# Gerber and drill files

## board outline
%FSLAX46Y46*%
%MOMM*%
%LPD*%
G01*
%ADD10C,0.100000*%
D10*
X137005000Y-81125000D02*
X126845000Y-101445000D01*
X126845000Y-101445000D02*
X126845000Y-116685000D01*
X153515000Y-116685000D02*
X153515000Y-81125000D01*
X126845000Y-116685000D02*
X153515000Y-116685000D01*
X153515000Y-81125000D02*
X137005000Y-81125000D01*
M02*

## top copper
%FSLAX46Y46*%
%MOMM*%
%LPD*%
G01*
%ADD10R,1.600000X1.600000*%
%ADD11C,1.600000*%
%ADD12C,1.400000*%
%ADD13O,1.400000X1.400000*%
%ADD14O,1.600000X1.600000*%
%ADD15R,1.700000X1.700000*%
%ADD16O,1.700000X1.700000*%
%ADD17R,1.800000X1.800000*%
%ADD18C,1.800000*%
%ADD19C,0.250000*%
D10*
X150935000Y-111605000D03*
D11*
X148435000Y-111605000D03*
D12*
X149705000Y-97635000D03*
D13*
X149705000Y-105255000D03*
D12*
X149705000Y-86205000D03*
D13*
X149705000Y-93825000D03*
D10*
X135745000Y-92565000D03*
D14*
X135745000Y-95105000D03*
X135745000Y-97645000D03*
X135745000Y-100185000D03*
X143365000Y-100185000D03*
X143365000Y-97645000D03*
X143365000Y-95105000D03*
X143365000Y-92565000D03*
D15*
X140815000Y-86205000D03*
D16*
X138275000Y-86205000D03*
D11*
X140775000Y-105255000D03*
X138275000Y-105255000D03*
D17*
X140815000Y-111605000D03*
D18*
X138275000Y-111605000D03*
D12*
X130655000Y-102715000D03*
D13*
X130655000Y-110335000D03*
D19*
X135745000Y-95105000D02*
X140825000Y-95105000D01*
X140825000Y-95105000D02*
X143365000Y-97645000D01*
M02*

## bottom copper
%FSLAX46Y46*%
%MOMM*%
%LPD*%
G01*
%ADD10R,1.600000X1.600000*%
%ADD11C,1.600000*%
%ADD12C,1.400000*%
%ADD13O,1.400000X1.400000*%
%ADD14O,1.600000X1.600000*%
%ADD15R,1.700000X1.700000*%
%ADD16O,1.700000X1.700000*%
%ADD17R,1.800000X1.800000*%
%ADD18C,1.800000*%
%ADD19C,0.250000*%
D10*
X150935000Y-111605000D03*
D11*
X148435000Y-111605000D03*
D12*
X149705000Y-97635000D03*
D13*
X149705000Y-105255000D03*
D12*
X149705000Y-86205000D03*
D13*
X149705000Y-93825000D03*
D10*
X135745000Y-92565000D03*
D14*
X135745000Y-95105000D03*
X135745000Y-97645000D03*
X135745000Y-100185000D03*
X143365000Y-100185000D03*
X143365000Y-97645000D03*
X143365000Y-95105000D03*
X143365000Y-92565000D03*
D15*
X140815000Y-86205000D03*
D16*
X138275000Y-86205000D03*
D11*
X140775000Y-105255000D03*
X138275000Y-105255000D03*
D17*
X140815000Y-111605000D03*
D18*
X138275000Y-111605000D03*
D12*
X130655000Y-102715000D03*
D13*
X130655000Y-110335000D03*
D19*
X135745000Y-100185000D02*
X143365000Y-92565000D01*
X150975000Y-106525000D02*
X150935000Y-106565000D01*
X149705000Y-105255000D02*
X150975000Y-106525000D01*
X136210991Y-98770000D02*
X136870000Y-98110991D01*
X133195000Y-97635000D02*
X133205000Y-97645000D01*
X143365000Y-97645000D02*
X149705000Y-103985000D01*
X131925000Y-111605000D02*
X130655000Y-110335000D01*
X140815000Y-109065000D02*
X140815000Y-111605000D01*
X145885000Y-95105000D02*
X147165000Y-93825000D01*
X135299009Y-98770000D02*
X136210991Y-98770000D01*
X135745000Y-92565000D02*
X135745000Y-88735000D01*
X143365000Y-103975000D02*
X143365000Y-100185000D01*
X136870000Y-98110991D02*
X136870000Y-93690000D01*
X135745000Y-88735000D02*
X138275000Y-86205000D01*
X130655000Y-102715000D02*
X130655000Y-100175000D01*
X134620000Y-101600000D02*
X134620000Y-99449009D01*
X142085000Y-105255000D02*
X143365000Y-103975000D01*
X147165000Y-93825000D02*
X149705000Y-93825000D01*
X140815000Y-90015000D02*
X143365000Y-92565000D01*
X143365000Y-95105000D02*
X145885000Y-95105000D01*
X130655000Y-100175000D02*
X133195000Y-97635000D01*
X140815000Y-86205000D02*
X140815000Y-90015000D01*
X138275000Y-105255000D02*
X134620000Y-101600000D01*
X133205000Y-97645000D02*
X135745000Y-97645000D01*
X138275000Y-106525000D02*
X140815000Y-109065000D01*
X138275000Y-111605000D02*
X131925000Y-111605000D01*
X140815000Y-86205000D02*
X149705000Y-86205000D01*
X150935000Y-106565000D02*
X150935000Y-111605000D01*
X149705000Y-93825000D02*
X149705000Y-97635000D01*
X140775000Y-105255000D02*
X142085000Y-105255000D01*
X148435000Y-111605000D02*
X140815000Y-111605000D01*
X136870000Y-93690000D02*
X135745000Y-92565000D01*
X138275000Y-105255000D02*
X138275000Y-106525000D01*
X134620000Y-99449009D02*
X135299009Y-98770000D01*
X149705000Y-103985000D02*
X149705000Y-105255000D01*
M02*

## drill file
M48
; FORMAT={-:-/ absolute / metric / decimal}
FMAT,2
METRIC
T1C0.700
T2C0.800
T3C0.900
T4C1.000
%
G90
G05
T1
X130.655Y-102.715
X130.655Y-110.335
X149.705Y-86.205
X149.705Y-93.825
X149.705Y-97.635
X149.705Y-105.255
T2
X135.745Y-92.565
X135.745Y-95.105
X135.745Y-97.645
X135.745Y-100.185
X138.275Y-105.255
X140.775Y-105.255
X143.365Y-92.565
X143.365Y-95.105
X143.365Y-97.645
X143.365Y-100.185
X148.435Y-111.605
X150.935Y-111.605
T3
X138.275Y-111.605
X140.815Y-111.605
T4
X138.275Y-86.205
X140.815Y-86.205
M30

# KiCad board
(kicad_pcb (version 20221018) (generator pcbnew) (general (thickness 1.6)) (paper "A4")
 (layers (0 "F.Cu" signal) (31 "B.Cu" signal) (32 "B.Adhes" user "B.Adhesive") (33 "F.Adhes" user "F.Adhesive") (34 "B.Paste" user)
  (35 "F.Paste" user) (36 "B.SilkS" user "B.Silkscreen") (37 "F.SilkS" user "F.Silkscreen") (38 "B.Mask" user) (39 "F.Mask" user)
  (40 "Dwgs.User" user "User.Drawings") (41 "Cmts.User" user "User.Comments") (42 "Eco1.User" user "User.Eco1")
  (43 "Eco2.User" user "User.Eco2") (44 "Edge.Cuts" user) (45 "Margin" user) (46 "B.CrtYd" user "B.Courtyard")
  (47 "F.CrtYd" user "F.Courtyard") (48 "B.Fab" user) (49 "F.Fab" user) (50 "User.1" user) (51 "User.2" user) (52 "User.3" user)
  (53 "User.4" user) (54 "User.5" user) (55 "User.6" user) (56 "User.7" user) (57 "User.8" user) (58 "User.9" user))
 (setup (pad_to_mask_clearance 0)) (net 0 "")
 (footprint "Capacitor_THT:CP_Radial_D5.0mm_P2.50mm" (layer "F.Cu") (at 150.935 111.605 180)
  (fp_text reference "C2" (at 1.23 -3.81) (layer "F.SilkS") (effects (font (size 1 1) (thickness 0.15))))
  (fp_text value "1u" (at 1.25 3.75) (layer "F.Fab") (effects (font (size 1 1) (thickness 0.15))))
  (pad "1" thru_hole rect (at 0 0 180) (size 1.6 1.6) (drill 0.8) (layers "*.Cu" "*.Mask"))
  (pad "2" thru_hole circle (at 2.5 0 180) (size 1.6 1.6) (drill 0.8) (layers "*.Cu" "*.Mask")))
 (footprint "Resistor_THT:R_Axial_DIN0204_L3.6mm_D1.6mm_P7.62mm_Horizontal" (layer "F.Cu") (at 149.705 97.635 -90)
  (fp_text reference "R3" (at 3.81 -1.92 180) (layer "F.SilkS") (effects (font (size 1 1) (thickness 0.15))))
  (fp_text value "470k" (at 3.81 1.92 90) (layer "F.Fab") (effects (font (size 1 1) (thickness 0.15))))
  (pad "1" thru_hole circle (at 0 0 270) (size 1.4 1.4) (drill 0.7) (layers "*.Cu" "*.Mask"))
  (pad "2" thru_hole oval (at 7.62 0 270) (size 1.4 1.4) (drill 0.7) (layers "*.Cu" "*.Mask")))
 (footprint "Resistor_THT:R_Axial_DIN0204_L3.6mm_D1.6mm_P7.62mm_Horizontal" (layer "F.Cu") (at 149.705 86.205 -90)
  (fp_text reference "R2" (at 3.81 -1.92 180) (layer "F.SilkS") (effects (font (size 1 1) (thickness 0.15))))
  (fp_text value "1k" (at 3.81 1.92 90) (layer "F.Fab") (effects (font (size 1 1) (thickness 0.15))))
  (pad "1" thru_hole circle (at 0 0 270) (size 1.4 1.4) (drill 0.7) (layers "*.Cu" "*.Mask"))
  (pad "2" thru_hole oval (at 7.62 0 270) (size 1.4 1.4) (drill 0.7) (layers "*.Cu" "*.Mask")))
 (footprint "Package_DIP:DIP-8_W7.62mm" (layer "F.Cu") (at 135.745 92.565)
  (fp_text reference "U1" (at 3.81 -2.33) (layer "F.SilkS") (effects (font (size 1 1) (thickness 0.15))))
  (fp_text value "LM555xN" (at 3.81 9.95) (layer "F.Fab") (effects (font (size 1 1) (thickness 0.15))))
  (pad "1" thru_hole rect (at 0 0) (size 1.6 1.6) (drill 0.8) (layers "*.Cu" "*.Mask"))
  (pad "2" thru_hole oval (at 0 2.54) (size 1.6 1.6) (drill 0.8) (layers "*.Cu" "*.Mask"))
  (pad "3" thru_hole oval (at 0 5.08) (size 1.6 1.6) (drill 0.8) (layers "*.Cu" "*.Mask"))
  (pad "4" thru_hole oval (at 0 7.62) (size 1.6 1.6) (drill 0.8) (layers "*.Cu" "*.Mask"))
  (pad "5" thru_hole oval (at 7.62 7.62) (size 1.6 1.6) (drill 0.8) (layers "*.Cu" "*.Mask"))
  (pad "6" thru_hole oval (at 7.62 5.08) (size 1.6 1.6) (drill 0.8) (layers "*.Cu" "*.Mask"))
  (pad "7" thru_hole oval (at 7.62 2.54) (size 1.6 1.6) (drill 0.8) (layers "*.Cu" "*.Mask"))
  (pad "8" thru_hole oval (at 7.62 0) (size 1.6 1.6) (drill 0.8) (layers "*.Cu" "*.Mask")))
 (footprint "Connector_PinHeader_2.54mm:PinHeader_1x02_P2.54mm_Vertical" (layer "F.Cu") (at 140.815 86.205 -90)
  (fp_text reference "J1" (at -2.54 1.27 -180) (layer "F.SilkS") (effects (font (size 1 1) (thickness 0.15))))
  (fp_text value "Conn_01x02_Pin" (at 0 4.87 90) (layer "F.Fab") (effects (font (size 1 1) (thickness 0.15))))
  (pad "1" thru_hole rect (at 0 0 270) (size 1.7 1.7) (drill 1) (layers "*.Cu" "*.Mask"))
  (pad "2" thru_hole oval (at 0 2.54 270) (size 1.7 1.7) (drill 1) (layers "*.Cu" "*.Mask")))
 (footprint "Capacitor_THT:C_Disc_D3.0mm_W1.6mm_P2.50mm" (layer "F.Cu") (at 140.775 105.255 180)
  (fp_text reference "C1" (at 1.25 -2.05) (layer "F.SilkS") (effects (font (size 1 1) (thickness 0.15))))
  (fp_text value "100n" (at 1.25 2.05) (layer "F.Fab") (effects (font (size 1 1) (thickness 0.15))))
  (pad "1" thru_hole circle (at 0 0 180) (size 1.6 1.6) (drill 0.8) (layers "*.Cu" "*.Mask"))
  (pad "2" thru_hole circle (at 2.5 0 180) (size 1.6 1.6) (drill 0.8) (layers "*.Cu" "*.Mask")))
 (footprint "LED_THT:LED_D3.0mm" (layer "F.Cu") (at 140.815 111.605 180)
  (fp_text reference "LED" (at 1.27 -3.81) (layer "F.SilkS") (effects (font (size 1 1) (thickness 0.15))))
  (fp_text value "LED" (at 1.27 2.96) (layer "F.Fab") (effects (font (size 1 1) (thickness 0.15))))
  (pad "1" thru_hole rect (at 0 0 180) (size 1.8 1.8) (drill 0.9) (layers "*.Cu" "*.Mask"))
  (pad "2" thru_hole circle (at 2.54 0 180) (size 1.8 1.8) (drill 0.9) (layers "*.Cu" "*.Mask")))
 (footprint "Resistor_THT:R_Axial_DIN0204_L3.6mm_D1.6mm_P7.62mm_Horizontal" (layer "F.Cu") (at 130.655 102.715 -90)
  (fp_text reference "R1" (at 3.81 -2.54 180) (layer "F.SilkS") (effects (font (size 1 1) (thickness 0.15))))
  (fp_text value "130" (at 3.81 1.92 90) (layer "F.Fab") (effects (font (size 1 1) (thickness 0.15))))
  (pad "1" thru_hole circle (at 0 0 270) (size 1.4 1.4) (drill 0.7) (layers "*.Cu" "*.Mask"))
  (pad "2" thru_hole oval (at 7.62 0 270) (size 1.4 1.4) (drill 0.7) (layers "*.Cu" "*.Mask")))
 (gr_line (start 137.005 81.125) (end 126.845 101.445) (stroke (width 0.1) (type default)) (layer "Edge.Cuts"))
 (gr_line (start 126.845 101.445) (end 126.845 116.685) (stroke (width 0.1) (type default)) (layer "Edge.Cuts"))
 (gr_line (start 153.515 116.685) (end 153.515 81.125) (stroke (width 0.1) (type default)) (layer "Edge.Cuts"))
 (gr_line (start 126.845 116.685) (end 153.515 116.685) (stroke (width 0.1) (type default)) (layer "Edge.Cuts"))
 (gr_line (start 153.515 81.125) (end 137.005 81.125) (stroke (width 0.1) (type default)) (layer "Edge.Cuts"))
 (segment (start 135.745 95.105) (end 140.825 95.105) (width 0.25) (layer "F.Cu") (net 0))
 (segment (start 140.825 95.105) (end 143.365 97.645) (width 0.25) (layer "F.Cu") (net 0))
 (segment (start 135.745 100.185) (end 143.365 92.565) (width 0.25) (layer "B.Cu") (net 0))
 (segment (start 150.975 106.525) (end 150.935 106.565) (width 0.25) (layer "B.Cu") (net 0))
 (segment (start 149.705 105.255) (end 150.975 106.525) (width 0.25) (layer "B.Cu") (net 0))
 (segment (start 136.210991 98.77) (end 136.87 98.110991) (width 0.25) (layer "B.Cu") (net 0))
 (segment (start 133.195 97.635) (end 133.205 97.645) (width 0.25) (layer "B.Cu") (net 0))
 (segment (start 143.365 97.645) (end 149.705 103.985) (width 0.25) (layer "B.Cu") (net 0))
 (segment (start 131.925 111.605) (end 130.655 110.335) (width 0.25) (layer "B.Cu") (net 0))
 (segment (start 140.815 109.065) (end 140.815 111.605) (width 0.25) (layer "B.Cu") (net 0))
 (segment (start 145.885 95.105) (end 147.165 93.825) (width 0.25) (layer "B.Cu") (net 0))
 (segment (start 135.299009 98.77) (end 136.210991 98.77) (width 0.25) (layer "B.Cu") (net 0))
 (segment (start 135.745 92.565) (end 135.745 88.735) (width 0.25) (layer "B.Cu") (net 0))
 (segment (start 143.365 103.975) (end 143.365 100.185) (width 0.25) (layer "B.Cu") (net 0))
 (segment (start 136.87 98.110991) (end 136.87 93.69) (width 0.25) (layer "B.Cu") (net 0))
 (segment (start 135.745 88.735) (end 138.275 86.205) (width 0.25) (layer "B.Cu") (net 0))
 (segment (start 130.655 102.715) (end 130.655 100.175) (width 0.25) (layer "B.Cu") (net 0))
 (segment (start 134.62 101.6) (end 134.62 99.449009) (width 0.25) (layer "B.Cu") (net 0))
 (segment (start 142.085 105.255) (end 143.365 103.975) (width 0.25) (layer "B.Cu") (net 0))
 (segment (start 147.165 93.825) (end 149.705 93.825) (width 0.25) (layer "B.Cu") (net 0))
 (segment (start 140.815 90.015) (end 143.365 92.565) (width 0.25) (layer "B.Cu") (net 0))
 (segment (start 143.365 95.105) (end 145.885 95.105) (width 0.25) (layer "B.Cu") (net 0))
 (segment (start 130.655 100.175) (end 133.195 97.635) (width 0.25) (layer "B.Cu") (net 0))
 (segment (start 140.815 86.205) (end 140.815 90.015) (width 0.25) (layer "B.Cu") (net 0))
 (segment (start 138.275 105.255) (end 134.62 101.6) (width 0.25) (layer "B.Cu") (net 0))
 (segment (start 133.205 97.645) (end 135.745 97.645) (width 0.25) (layer "B.Cu") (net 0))
 (segment (start 138.275 106.525) (end 140.815 109.065) (width 0.25) (layer "B.Cu") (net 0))
 (segment (start 138.275 111.605) (end 131.925 111.605) (width 0.25) (layer "B.Cu") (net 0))
 (segment (start 140.815 86.205) (end 149.705 86.205) (width 0.25) (layer "B.Cu") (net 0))
 (segment (start 150.935 106.565) (end 150.935 111.605) (width 0.25) (layer "B.Cu") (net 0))
 (segment (start 149.705 93.825) (end 149.705 97.635) (width 0.25) (layer "B.Cu") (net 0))
 (segment (start 140.775 105.255) (end 142.085 105.255) (width 0.25) (layer "B.Cu") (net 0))
 (segment (start 148.435 111.605) (end 140.815 111.605) (width 0.25) (layer "B.Cu") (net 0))
 (segment (start 136.87 93.69) (end 135.745 92.565) (width 0.25) (layer "B.Cu") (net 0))
 (segment (start 138.275 105.255) (end 138.275 106.525) (width 0.25) (layer "B.Cu") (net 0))
 (segment (start 134.62 99.449009) (end 135.299009 98.77) (width 0.25) (layer "B.Cu") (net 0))
 (segment (start 149.705 103.985) (end 149.705 105.255) (width 0.25) (layer "B.Cu") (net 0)))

